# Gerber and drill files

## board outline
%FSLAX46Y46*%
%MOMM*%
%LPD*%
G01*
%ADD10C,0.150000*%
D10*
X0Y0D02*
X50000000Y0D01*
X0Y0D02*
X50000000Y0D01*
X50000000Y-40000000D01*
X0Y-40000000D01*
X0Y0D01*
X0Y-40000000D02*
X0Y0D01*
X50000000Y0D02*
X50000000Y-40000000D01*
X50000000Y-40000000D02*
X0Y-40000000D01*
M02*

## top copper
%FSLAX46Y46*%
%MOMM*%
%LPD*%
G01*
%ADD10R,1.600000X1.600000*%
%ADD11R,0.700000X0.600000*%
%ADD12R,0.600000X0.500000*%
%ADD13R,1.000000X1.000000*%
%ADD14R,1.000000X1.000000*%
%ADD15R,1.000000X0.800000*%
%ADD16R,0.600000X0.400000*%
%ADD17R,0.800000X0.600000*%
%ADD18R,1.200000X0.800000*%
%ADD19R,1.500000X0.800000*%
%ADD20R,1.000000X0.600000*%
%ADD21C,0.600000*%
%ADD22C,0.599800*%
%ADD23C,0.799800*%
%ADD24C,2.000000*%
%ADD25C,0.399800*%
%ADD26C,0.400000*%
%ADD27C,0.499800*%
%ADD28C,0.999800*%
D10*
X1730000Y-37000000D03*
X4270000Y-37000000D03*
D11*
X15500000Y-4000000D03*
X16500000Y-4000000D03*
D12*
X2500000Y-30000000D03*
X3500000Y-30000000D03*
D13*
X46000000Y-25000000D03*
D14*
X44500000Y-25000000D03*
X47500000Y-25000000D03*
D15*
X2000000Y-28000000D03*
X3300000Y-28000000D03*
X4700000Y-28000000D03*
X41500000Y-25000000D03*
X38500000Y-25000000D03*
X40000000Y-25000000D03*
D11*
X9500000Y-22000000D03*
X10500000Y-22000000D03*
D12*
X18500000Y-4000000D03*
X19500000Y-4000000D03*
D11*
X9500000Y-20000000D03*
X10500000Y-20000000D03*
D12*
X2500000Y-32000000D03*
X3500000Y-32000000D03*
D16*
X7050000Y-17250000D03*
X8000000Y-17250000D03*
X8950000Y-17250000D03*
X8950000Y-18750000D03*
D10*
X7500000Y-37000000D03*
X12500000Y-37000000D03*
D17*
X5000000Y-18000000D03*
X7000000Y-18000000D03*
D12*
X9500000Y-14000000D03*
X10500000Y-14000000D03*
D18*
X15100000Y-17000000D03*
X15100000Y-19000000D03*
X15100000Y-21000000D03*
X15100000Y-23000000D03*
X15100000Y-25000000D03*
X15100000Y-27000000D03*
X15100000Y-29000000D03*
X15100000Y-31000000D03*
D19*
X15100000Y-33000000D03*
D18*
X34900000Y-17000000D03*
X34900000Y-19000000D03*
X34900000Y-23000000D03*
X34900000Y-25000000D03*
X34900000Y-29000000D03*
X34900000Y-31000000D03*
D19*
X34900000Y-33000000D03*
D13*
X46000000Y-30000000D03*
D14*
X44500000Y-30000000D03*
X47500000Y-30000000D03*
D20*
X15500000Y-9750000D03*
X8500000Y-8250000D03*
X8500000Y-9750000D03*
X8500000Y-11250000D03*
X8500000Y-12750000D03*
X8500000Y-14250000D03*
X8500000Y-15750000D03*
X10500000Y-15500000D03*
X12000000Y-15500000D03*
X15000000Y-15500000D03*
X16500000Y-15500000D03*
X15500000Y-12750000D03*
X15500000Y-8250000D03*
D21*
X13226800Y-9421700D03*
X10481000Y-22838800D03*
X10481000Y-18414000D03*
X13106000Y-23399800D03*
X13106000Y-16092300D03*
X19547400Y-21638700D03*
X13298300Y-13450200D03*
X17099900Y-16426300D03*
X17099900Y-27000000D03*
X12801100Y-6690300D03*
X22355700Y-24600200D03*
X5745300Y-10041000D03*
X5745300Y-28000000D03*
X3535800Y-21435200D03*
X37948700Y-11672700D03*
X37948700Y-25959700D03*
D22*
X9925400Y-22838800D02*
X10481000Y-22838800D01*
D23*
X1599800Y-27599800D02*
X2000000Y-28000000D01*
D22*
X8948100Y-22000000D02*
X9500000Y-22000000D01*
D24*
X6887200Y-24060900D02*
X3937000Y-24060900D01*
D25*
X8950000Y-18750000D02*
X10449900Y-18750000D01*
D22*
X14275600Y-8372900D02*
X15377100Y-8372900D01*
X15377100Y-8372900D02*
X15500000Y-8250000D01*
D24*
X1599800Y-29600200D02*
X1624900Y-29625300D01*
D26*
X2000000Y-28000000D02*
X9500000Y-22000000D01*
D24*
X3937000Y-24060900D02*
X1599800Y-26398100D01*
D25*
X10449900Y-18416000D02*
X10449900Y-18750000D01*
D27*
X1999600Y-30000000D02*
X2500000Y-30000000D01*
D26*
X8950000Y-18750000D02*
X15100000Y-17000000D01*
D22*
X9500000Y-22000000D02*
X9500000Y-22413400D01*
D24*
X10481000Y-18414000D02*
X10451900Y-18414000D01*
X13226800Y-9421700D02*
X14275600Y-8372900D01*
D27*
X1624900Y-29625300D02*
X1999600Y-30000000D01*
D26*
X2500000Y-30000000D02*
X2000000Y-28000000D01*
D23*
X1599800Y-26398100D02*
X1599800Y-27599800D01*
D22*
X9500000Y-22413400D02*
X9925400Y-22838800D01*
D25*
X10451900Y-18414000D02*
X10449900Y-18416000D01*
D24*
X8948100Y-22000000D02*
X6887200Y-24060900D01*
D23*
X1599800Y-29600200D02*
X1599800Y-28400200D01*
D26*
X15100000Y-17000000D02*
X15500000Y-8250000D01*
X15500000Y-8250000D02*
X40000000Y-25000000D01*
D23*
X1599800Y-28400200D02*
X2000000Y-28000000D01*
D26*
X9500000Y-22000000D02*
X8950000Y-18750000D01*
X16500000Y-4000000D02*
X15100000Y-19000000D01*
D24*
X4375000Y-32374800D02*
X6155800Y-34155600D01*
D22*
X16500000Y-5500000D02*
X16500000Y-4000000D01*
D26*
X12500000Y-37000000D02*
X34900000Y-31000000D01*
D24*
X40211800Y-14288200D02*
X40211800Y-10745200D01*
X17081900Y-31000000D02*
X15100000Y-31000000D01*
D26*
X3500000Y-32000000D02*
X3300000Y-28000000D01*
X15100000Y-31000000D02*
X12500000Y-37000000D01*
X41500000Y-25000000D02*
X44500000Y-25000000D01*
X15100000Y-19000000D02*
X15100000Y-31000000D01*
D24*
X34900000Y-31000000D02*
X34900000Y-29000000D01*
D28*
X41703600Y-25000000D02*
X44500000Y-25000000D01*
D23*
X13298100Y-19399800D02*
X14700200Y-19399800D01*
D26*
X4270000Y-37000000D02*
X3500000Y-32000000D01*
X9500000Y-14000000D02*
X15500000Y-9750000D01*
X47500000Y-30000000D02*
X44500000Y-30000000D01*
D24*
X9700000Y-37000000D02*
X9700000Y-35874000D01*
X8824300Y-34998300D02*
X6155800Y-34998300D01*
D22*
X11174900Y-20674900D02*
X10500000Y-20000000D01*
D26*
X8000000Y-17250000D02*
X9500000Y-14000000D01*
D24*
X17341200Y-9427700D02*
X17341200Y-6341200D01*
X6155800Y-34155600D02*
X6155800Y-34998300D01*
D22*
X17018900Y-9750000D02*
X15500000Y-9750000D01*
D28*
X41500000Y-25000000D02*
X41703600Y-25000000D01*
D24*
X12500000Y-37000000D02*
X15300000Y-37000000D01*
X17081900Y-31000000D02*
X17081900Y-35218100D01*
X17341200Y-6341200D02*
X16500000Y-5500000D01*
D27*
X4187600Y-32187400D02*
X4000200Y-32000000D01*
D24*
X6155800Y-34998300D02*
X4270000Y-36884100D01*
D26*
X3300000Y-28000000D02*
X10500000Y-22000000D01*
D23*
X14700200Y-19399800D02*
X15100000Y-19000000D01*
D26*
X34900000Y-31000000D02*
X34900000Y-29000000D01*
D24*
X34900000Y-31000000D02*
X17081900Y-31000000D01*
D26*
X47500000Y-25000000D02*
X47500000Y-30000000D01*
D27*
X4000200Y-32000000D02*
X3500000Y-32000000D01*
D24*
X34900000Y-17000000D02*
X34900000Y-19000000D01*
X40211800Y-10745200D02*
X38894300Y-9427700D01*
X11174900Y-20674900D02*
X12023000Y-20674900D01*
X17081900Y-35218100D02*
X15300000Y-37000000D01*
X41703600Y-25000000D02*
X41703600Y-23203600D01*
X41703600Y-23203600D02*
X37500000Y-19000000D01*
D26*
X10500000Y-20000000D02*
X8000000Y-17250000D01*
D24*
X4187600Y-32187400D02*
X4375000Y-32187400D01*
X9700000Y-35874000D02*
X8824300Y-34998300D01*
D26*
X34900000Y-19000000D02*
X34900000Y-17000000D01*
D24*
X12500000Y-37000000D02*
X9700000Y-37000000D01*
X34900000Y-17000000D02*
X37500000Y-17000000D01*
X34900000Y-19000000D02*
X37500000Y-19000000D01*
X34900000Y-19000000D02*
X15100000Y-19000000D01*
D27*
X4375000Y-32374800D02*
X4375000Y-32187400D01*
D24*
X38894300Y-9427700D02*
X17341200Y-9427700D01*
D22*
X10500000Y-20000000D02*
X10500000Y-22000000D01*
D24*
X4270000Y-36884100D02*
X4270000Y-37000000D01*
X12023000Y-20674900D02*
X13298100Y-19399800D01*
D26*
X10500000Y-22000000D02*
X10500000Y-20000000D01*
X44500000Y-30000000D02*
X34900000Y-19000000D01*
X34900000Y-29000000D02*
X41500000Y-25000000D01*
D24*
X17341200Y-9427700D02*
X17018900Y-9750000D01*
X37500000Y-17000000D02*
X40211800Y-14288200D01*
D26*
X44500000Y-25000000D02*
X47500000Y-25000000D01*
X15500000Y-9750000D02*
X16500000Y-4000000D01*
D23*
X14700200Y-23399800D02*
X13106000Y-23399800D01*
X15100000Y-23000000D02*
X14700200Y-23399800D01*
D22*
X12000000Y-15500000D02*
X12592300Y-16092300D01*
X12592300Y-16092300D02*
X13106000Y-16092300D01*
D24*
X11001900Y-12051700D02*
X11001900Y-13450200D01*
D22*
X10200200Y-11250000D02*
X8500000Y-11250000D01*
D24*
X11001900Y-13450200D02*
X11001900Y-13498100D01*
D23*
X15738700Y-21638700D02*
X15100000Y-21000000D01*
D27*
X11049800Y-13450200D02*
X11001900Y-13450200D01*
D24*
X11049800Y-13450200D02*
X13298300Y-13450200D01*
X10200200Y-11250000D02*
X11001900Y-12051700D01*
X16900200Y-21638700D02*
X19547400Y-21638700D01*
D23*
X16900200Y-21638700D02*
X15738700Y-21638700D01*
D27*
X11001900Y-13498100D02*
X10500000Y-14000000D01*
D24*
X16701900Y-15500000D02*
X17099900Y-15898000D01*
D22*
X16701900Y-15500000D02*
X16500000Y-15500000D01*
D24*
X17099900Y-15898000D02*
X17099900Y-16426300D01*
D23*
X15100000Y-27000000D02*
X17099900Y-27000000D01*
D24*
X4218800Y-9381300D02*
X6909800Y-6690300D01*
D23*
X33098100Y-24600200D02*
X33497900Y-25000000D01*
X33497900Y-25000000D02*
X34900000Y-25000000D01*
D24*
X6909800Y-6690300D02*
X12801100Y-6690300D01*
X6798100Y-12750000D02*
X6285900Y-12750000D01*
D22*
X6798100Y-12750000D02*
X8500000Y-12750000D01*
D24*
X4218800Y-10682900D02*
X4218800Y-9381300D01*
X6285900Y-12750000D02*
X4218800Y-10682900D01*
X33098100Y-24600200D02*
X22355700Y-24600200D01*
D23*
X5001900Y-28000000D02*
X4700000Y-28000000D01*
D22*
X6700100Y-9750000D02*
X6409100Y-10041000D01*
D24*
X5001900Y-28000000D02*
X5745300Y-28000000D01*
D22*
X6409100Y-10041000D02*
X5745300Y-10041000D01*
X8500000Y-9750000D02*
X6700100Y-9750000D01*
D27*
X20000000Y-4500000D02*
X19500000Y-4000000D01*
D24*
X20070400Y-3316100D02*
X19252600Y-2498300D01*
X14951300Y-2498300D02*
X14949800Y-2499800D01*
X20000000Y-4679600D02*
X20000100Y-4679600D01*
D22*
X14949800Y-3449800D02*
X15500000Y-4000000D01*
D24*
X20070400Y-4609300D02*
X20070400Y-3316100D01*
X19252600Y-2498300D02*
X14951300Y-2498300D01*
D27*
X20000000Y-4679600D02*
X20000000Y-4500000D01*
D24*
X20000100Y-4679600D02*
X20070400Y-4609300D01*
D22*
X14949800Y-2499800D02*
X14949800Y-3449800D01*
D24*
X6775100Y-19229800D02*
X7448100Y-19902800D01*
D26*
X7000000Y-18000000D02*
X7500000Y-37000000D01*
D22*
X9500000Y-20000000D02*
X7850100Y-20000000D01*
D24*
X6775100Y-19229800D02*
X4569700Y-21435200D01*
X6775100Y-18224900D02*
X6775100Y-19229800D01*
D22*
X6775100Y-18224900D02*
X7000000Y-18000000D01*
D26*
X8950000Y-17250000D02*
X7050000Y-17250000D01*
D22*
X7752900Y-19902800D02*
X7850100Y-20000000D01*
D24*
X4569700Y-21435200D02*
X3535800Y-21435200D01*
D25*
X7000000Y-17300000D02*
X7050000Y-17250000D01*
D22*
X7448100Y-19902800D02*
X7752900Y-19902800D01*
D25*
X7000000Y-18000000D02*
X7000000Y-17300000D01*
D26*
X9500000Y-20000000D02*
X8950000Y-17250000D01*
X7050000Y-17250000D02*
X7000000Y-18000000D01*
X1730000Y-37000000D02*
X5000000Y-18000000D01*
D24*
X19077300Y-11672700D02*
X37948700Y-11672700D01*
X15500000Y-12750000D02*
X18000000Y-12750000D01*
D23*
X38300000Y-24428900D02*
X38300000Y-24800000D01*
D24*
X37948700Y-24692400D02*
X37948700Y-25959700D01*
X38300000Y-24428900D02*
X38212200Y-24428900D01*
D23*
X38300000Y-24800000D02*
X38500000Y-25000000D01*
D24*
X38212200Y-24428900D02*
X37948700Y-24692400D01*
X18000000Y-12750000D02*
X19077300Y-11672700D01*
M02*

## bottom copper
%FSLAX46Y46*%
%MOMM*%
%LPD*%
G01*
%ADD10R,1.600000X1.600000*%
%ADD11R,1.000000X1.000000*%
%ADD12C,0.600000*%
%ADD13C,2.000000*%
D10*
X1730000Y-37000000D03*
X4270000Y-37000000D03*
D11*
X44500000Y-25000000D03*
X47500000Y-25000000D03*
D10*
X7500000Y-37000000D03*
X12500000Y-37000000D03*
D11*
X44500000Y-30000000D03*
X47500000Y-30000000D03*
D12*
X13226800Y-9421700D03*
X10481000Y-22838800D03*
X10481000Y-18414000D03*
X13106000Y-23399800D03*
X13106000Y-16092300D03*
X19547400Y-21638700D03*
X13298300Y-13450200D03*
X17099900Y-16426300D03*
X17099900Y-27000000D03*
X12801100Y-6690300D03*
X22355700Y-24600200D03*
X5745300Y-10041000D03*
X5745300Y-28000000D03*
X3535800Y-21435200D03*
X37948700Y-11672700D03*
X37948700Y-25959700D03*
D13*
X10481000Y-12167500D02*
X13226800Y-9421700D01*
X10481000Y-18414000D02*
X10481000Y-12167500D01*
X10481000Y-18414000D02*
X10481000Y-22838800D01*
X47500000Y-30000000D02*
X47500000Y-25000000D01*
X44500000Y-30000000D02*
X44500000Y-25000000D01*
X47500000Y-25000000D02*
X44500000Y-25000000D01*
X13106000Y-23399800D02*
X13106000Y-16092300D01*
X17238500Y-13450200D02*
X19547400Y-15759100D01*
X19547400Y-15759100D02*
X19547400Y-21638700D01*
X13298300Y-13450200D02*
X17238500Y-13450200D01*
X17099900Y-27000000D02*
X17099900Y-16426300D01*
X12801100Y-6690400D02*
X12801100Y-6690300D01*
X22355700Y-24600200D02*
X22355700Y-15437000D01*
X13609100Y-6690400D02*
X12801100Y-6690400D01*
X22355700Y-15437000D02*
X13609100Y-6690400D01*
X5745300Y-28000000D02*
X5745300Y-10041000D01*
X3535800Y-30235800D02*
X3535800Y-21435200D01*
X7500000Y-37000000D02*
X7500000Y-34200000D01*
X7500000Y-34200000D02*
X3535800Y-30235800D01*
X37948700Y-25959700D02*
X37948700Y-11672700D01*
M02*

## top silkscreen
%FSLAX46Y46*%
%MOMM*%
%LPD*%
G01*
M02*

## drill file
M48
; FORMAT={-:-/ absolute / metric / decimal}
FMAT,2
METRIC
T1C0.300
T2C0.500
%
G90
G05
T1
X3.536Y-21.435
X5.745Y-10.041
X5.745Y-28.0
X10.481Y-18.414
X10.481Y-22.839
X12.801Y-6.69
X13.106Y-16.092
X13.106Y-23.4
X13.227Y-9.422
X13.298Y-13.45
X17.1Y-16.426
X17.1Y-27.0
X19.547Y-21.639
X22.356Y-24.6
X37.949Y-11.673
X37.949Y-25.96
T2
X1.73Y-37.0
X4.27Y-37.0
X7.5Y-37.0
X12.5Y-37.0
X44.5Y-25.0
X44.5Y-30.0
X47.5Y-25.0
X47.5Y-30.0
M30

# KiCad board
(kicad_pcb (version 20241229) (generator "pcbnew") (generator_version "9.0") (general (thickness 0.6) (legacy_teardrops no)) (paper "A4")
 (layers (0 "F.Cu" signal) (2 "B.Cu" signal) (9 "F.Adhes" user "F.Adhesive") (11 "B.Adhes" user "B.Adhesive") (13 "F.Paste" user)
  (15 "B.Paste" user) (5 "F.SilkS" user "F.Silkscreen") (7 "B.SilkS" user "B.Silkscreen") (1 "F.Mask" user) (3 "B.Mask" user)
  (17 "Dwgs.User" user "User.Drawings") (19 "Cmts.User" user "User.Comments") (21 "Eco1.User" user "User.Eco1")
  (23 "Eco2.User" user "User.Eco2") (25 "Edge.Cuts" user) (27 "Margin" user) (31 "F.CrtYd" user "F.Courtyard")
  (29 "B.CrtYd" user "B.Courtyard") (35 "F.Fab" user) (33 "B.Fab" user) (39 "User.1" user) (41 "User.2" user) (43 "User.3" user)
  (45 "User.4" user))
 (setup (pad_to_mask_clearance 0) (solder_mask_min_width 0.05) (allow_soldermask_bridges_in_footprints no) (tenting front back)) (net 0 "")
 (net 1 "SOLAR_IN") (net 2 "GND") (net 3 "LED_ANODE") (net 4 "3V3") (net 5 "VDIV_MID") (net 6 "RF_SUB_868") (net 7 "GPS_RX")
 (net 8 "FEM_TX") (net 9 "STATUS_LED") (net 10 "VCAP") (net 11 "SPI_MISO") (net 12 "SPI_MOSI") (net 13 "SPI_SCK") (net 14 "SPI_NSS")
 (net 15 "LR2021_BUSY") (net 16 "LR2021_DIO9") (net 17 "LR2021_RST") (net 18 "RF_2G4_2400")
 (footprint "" (layer "F.Cu") (at 3 37)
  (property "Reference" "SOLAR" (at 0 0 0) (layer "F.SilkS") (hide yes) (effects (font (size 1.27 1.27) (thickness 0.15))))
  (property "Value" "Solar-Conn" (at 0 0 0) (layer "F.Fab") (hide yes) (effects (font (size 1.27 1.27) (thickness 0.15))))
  (pad "1" thru_hole rect (at -1.27 0) (size 1.6 1.6) (drill 0.5) (layers "*.Cu" "*.Mask") (remove_unused_layers no) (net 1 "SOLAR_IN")
   (thermal_bridge_angle 45))
  (pad "2" thru_hole rect (at 1.27 0) (size 1.6 1.6) (drill 0.5) (layers "*.Cu" "*.Mask") (remove_unused_layers no) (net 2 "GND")
   (thermal_bridge_angle 45)))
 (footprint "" (layer "F.Cu") (at 16 4)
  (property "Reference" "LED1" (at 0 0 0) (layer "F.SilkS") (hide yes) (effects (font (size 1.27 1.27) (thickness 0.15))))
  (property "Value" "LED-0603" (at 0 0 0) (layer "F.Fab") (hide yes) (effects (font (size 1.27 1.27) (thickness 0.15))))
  (pad "A" smd rect (at -0.5 0) (size 0.7 0.6) (layers "F.Cu" "F.Mask") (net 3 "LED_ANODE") (thermal_bridge_angle 45))
  (pad "K" smd rect (at 0.5 0) (size 0.7 0.6) (layers "F.Cu" "F.Mask") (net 2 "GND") (thermal_bridge_angle 45)))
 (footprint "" (layer "F.Cu") (at 3 30)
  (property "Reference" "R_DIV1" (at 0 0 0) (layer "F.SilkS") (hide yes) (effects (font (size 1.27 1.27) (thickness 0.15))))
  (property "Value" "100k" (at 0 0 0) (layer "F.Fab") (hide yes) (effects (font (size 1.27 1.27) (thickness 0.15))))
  (pad "1" smd rect (at -0.5 0) (size 0.6 0.5) (layers "F.Cu" "F.Mask") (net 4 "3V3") (thermal_bridge_angle 45))
  (pad "2" smd rect (at 0.5 0) (size 0.6 0.5) (layers "F.Cu" "F.Mask") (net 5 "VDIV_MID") (thermal_bridge_angle 45)))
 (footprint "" (layer "F.Cu") (at 46 25)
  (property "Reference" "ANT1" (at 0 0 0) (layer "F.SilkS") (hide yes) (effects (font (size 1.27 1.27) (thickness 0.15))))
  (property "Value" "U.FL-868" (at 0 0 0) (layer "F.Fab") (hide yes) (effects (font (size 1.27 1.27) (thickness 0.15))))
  (pad "1" smd rect (at 0 0) (size 1 1) (layers "F.Cu" "F.Mask") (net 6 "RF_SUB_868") (thermal_bridge_angle 45))
  (pad "2" thru_hole rect (at -1.5 0) (size 1 1) (drill 0.5) (layers "*.Cu" "*.Mask") (remove_unused_layers no) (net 2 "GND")
   (thermal_bridge_angle 45))
  (pad "3" thru_hole rect (at 1.5 0) (size 1 1) (drill 0.5) (layers "*.Cu" "*.Mask") (remove_unused_layers no) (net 2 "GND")
   (thermal_bridge_angle 45)))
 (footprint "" (layer "F.Cu") (at 4 28)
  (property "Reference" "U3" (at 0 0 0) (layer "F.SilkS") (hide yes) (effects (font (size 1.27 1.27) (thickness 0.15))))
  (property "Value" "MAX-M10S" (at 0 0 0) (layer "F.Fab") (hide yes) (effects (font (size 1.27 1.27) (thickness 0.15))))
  (pad "1" smd rect (at -2 0) (size 1 0.8) (layers "F.Cu" "F.Mask") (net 4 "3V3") (thermal_bridge_angle 45))
  (pad "2" smd rect (at -0.7 0) (size 1 0.8) (layers "F.Cu" "F.Mask") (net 2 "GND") (thermal_bridge_angle 45))
  (pad "3" smd rect (at 0.7 0) (size 1 0.8) (layers "F.Cu" "F.Mask") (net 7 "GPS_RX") (thermal_bridge_angle 45)))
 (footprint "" (layer "F.Cu") (at 40 25)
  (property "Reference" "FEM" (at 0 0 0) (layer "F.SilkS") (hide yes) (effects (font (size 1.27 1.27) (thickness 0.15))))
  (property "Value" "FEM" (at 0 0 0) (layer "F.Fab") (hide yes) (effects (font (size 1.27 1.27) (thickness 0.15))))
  (pad "GND" smd rect (at 1.5 0) (size 1 0.8) (layers "F.Cu" "F.Mask") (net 2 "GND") (thermal_bridge_angle 45))
  (pad "TX" smd rect (at -1.5 0) (size 1 0.8) (layers "F.Cu" "F.Mask") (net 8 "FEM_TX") (thermal_bridge_angle 45))
  (pad "VCC" smd rect (at 0 0) (size 1 0.8) (layers "F.Cu" "F.Mask") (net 4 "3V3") (thermal_bridge_angle 45)))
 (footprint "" (layer "F.Cu") (at 10 22)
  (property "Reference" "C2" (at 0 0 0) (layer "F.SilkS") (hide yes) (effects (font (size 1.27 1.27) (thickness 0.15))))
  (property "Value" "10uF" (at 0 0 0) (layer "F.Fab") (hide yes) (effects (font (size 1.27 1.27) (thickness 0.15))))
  (pad "1" smd rect (at -0.5 0) (size 0.7 0.6) (layers "F.Cu" "F.Mask") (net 4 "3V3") (thermal_bridge_angle 45))
  (pad "2" smd rect (at 0.5 0) (size 0.7 0.6) (layers "F.Cu" "F.Mask") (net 2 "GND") (thermal_bridge_angle 45)))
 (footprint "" (layer "F.Cu") (at 19 4)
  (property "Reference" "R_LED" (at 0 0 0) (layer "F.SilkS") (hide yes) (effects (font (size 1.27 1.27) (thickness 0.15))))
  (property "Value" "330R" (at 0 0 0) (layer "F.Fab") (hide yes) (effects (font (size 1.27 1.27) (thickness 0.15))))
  (pad "1" smd rect (at -0.5 0) (size 0.6 0.5) (layers "F.Cu" "F.Mask") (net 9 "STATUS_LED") (thermal_bridge_angle 45))
  (pad "2" smd rect (at 0.5 0) (size 0.6 0.5) (layers "F.Cu" "F.Mask") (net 3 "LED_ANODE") (thermal_bridge_angle 45)))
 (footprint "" (layer "F.Cu") (at 10 20)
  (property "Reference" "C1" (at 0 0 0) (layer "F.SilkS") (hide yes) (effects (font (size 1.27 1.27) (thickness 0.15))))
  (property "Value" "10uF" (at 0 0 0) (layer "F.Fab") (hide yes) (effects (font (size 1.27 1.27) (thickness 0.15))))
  (pad "1" smd rect (at -0.5 0) (size 0.7 0.6) (layers "F.Cu" "F.Mask") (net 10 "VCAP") (thermal_bridge_angle 45))
  (pad "2" smd rect (at 0.5 0) (size 0.7 0.6) (layers "F.Cu" "F.Mask") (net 2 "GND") (thermal_bridge_angle 45)))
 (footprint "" (layer "F.Cu") (at 3 32)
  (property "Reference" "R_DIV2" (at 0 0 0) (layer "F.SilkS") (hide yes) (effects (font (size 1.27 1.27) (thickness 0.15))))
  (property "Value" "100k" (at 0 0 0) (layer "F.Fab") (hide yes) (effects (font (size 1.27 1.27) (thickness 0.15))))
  (pad "1" smd rect (at -0.5 0) (size 0.6 0.5) (layers "F.Cu" "F.Mask") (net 5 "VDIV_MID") (thermal_bridge_angle 45))
  (pad "2" smd rect (at 0.5 0) (size 0.6 0.5) (layers "F.Cu" "F.Mask") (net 2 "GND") (thermal_bridge_angle 45)))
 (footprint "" (layer "F.Cu") (at 8 18)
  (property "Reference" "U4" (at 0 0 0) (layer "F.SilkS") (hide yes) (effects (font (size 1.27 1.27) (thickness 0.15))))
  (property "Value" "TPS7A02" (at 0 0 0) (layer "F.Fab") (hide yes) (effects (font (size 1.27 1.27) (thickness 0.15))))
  (pad "1" smd rect (at -0.95 -0.75) (size 0.6 0.4) (layers "F.Cu" "F.Mask") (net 10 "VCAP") (thermal_bridge_angle 45))
  (pad "2" smd rect (at 0 -0.75) (size 0.6 0.4) (layers "F.Cu" "F.Mask") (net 2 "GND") (thermal_bridge_angle 45))
  (pad "3" smd rect (at 0.95 -0.75) (size 0.6 0.4) (layers "F.Cu" "F.Mask") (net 10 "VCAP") (thermal_bridge_angle 45))
  (pad "4" smd rect (at 0.95 0.75) (size 0.6 0.4) (layers "F.Cu" "F.Mask") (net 4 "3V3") (thermal_bridge_angle 45)))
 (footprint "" (layer "F.Cu") (at 10 37)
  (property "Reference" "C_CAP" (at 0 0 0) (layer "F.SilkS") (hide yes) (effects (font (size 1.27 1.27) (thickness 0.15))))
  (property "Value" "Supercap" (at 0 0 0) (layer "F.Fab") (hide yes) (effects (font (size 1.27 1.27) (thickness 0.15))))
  (pad "1" thru_hole rect (at -2.5 0) (size 1.6 1.6) (drill 0.5) (layers "*.Cu" "*.Mask") (remove_unused_layers no) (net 10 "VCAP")
   (thermal_bridge_angle 45))
  (pad "2" thru_hole rect (at 2.5 0) (size 1.6 1.6) (drill 0.5) (layers "*.Cu" "*.Mask") (remove_unused_layers no) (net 2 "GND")
   (thermal_bridge_angle 45)))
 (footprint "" (layer "F.Cu") (at 6 18)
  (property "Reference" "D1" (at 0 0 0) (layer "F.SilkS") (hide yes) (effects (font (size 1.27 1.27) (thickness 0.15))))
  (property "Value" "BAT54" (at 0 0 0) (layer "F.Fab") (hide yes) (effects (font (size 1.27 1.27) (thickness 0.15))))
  (pad "A" smd rect (at -1 0) (size 0.8 0.6) (layers "F.Cu" "F.Mask") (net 1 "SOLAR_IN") (thermal_bridge_angle 45))
  (pad "K" smd rect (at 1 0) (size 0.8 0.6) (layers "F.Cu" "F.Mask") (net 10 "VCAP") (thermal_bridge_angle 45)))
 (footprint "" (layer "F.Cu") (at 10 14)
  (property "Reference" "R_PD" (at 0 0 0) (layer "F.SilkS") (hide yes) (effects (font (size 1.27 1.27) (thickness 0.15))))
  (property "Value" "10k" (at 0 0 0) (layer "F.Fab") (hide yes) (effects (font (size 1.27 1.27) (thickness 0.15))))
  (pad "1" smd rect (at -0.5 0) (size 0.6 0.5) (layers "F.Cu" "F.Mask") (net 2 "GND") (thermal_bridge_angle 45))
  (pad "2" smd rect (at 0.5 0) (size 0.6 0.5) (layers "F.Cu" "F.Mask") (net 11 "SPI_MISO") (thermal_bridge_angle 45)))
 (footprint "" (layer "F.Cu") (at 25 25)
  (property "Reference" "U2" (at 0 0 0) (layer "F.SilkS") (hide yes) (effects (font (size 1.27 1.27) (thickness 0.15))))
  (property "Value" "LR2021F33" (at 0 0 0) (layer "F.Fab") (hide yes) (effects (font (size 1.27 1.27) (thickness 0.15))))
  (pad "1" smd rect (at -9.9 -8) (size 1.2 0.8) (layers "F.Cu" "F.Mask") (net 4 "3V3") (thermal_bridge_angle 45))
  (pad "2" smd rect (at -9.9 -6) (size 1.2 0.8) (layers "F.Cu" "F.Mask") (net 2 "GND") (thermal_bridge_angle 45))
  (pad "3" smd rect (at -9.9 -4) (size 1.2 0.8) (layers "F.Cu" "F.Mask") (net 11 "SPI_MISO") (thermal_bridge_angle 45))
  (pad "4" smd rect (at -9.9 -2) (size 1.2 0.8) (layers "F.Cu" "F.Mask") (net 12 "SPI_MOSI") (thermal_bridge_angle 45))
  (pad "5" smd rect (at -9.9 0) (size 1.2 0.8) (layers "F.Cu" "F.Mask") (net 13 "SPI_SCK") (thermal_bridge_angle 45))
  (pad "6" smd rect (at -9.9 2) (size 1.2 0.8) (layers "F.Cu" "F.Mask") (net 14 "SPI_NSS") (thermal_bridge_angle 45))
  (pad "7" smd rect (at -9.9 4) (size 1.2 0.8) (layers "F.Cu" "F.Mask") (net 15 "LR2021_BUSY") (thermal_bridge_angle 45))
  (pad "8" smd rect (at -9.9 6) (size 1.2 0.8) (layers "F.Cu" "F.Mask") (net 2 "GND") (thermal_bridge_angle 45))
  (pad "9" smd rect (at -9.9 8) (size 1.5 0.8) (layers "F.Cu" "F.Mask") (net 6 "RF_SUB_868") (thermal_bridge_angle 45))
  (pad "10" smd rect (at 9.9 -8) (size 1.2 0.8) (layers "F.Cu" "F.Mask") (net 2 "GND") (thermal_bridge_angle 45))
  (pad "11" smd rect (at 9.9 -6) (size 1.2 0.8) (layers "F.Cu" "F.Mask") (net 2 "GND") (thermal_bridge_angle 45))
  (pad "13" smd rect (at 9.9 -2) (size 1.2 0.8) (layers "F.Cu" "F.Mask") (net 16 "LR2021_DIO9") (thermal_bridge_angle 45))
  (pad "14" smd rect (at 9.9 0) (size 1.2 0.8) (layers "F.Cu" "F.Mask") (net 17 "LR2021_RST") (thermal_bridge_angle 45))
  (pad "16" smd rect (at 9.9 4) (size 1.2 0.8) (layers "F.Cu" "F.Mask") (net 2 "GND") (thermal_bridge_angle 45))
  (pad "17" smd rect (at 9.9 6) (size 1.2 0.8) (layers "F.Cu" "F.Mask") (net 2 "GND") (thermal_bridge_angle 45))
  (pad "18" smd rect (at 9.9 8) (size 1.5 0.8) (layers "F.Cu" "F.Mask") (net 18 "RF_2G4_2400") (thermal_bridge_angle 45)))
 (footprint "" (layer "F.Cu") (at 46 30)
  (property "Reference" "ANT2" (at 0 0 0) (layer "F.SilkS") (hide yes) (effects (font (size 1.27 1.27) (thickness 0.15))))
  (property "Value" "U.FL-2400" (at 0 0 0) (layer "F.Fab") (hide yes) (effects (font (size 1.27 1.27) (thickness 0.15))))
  (pad "1" smd rect (at 0 0) (size 1 1) (layers "F.Cu" "F.Mask") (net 18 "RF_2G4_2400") (thermal_bridge_angle 45))
  (pad "2" thru_hole rect (at -1.5 0) (size 1 1) (drill 0.5) (layers "*.Cu" "*.Mask") (remove_unused_layers no) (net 2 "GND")
   (thermal_bridge_angle 45))
  (pad "3" thru_hole rect (at 1.5 0) (size 1 1) (drill 0.5) (layers "*.Cu" "*.Mask") (remove_unused_layers no) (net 2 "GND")
   (thermal_bridge_angle 45)))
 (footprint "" (layer "F.Cu") (at 12 12)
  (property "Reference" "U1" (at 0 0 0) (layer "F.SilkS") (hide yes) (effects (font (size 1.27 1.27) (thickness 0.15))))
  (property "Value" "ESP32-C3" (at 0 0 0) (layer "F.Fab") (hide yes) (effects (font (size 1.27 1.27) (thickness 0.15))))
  (pad "GND" smd rect (at 3.5 -2.25) (size 1 0.6) (layers "F.Cu" "F.Mask") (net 2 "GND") (thermal_bridge_angle 45))
  (pad "GPIO0" smd rect (at -3.5 -3.75) (size 1 0.6) (layers "F.Cu" "F.Mask") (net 5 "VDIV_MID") (thermal_bridge_angle 45))
  (pad "GPIO1" smd rect (at -3.5 -2.25) (size 1 0.6) (layers "F.Cu" "F.Mask") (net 7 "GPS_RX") (thermal_bridge_angle 45))
  (pad "GPIO2" smd rect (at -3.5 -0.75) (size 1 0.6) (layers "F.Cu" "F.Mask") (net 11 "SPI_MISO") (thermal_bridge_angle 45))
  (pad "GPIO3" smd rect (at -3.5 0.75) (size 1 0.6) (layers "F.Cu" "F.Mask") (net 17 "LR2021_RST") (thermal_bridge_angle 45))
  (pad "GPIO4" smd rect (at -3.5 2.25) (size 1 0.6) (layers "F.Cu" "F.Mask") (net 15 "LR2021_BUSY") (thermal_bridge_angle 45))
  (pad "GPIO5" smd rect (at -3.5 3.75) (size 1 0.6) (layers "F.Cu" "F.Mask") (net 16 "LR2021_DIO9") (thermal_bridge_angle 45))
  (pad "GPIO6" smd rect (at -1.5 3.5) (size 1 0.6) (layers "F.Cu" "F.Mask") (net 13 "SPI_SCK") (thermal_bridge_angle 45))
  (pad "GPIO7" smd rect (at 0 3.5) (size 1 0.6) (layers "F.Cu" "F.Mask") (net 12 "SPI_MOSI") (thermal_bridge_angle 45))
  (pad "GPIO9" smd rect (at 3 3.5) (size 1 0.6) (layers "F.Cu" "F.Mask") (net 9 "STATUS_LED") (thermal_bridge_angle 45))
  (pad "GPIO10" smd rect (at 4.5 3.5) (size 1 0.6) (layers "F.Cu" "F.Mask") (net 14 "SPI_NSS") (thermal_bridge_angle 45))
  (pad "GPIO19" smd rect (at 3.5 0.75) (size 1 0.6) (layers "F.Cu" "F.Mask") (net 8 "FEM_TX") (thermal_bridge_angle 45))
  (pad "VCC" smd rect (at 3.5 -3.75) (size 1 0.6) (layers "F.Cu" "F.Mask") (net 4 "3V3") (thermal_bridge_angle 45)))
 (gr_line (start 0 0) (end 50 0) (stroke (width 0.15) (type default)) (layer "Edge.Cuts"))
 (gr_rect (start 0 0) (end 50 40) (stroke (width 0.15) (type default)) (fill no) (layer "Edge.Cuts"))
 (gr_line (start 0 40) (end 0 0) (stroke (width 0.15) (type default)) (layer "Edge.Cuts"))
 (gr_line (start 50 0) (end 50 40) (stroke (width 0.15) (type default)) (layer "Edge.Cuts"))
 (gr_line (start 50 40) (end 0 40) (stroke (width 0.15) (type default)) (layer "Edge.Cuts"))
 (segment (start 9.9254 22.8388) (end 10.481 22.8388) (width 0.5998) (layer "F.Cu") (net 4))
 (segment (start 1.5998 27.5998) (end 2 28) (width 0.7998) (layer "F.Cu") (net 4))
 (segment (start 8.9481 22) (end 9.5 22) (width 0.5998) (layer "F.Cu") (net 4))
 (segment (start 6.8872 24.0609) (end 3.937 24.0609) (width 2) (layer "F.Cu") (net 4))
 (segment (start 8.95 18.75) (end 10.4499 18.75) (width 0.3998) (layer "F.Cu") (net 4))
 (segment (start 14.2756 8.3729) (end 15.3771 8.3729) (width 0.5998) (layer "F.Cu") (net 4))
 (segment (start 15.3771 8.3729) (end 15.5 8.25) (width 0.5998) (layer "F.Cu") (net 4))
 (segment (start 1.5998 29.6002) (end 1.6249 29.6253) (width 2) (layer "F.Cu") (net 4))
 (segment (start 2 28) (end 9.5 22) (width 0.4) (layer "F.Cu") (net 4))
 (segment (start 3.937 24.0609) (end 1.5998 26.3981) (width 2) (layer "F.Cu") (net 4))
 (segment (start 10.4499 18.416) (end 10.4499 18.75) (width 0.3998) (layer "F.Cu") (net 4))
 (segment (start 1.9996 30) (end 2.5 30) (width 0.4998) (layer "F.Cu") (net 4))
 (segment (start 8.95 18.75) (end 15.1 17) (width 0.4) (layer "F.Cu") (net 4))
 (segment (start 9.5 22) (end 9.5 22.4134) (width 0.5998) (layer "F.Cu") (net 4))
 (segment (start 10.481 18.414) (end 10.4519 18.414) (width 2) (layer "F.Cu") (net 4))
 (segment (start 13.2268 9.4217) (end 14.2756 8.3729) (width 2) (layer "F.Cu") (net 4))
 (segment (start 1.6249 29.6253) (end 1.9996 30) (width 0.4998) (layer "F.Cu") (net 4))
 (segment (start 2.5 30) (end 2 28) (width 0.4) (layer "F.Cu") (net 4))
 (segment (start 1.5998 26.3981) (end 1.5998 27.5998) (width 0.7998) (layer "F.Cu") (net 4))
 (segment (start 9.5 22.4134) (end 9.9254 22.8388) (width 0.5998) (layer "F.Cu") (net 4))
 (segment (start 10.4519 18.414) (end 10.4499 18.416) (width 0.3998) (layer "F.Cu") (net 4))
 (segment (start 8.9481 22) (end 6.8872 24.0609) (width 2) (layer "F.Cu") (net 4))
 (segment (start 1.5998 29.6002) (end 1.5998 28.4002) (width 0.7998) (layer "F.Cu") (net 4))
 (segment (start 15.1 17) (end 15.5 8.25) (width 0.4) (layer "F.Cu") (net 4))
 (segment (start 15.5 8.25) (end 40 25) (width 0.4) (layer "F.Cu") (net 4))
 (segment (start 1.5998 28.4002) (end 2 28) (width 0.7998) (layer "F.Cu") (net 4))
 (segment (start 9.5 22) (end 8.95 18.75) (width 0.4) (layer "F.Cu") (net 4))
 (via (at 13.2268 9.4217) (size 0.6) (drill 0.3) (layers "F.Cu" "B.Cu") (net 4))
 (via (at 10.481 22.8388) (size 0.6) (drill 0.3) (layers "F.Cu" "B.Cu") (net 4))
 (via (at 10.481 18.414) (size 0.6) (drill 0.3) (layers "F.Cu" "B.Cu") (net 4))
 (segment (start 10.481 12.1675) (end 13.2268 9.4217) (width 2) (layer "B.Cu") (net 4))
 (segment (start 10.481 18.414) (end 10.481 12.1675) (width 2) (layer "B.Cu") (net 4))
 (segment (start 10.481 18.414) (end 10.481 22.8388) (width 2) (layer "B.Cu") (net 4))
 (segment (start 16.5 4) (end 15.1 19) (width 0.4) (layer "F.Cu") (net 2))
 (segment (start 4.375 32.3748) (end 6.1558 34.1556) (width 2) (layer "F.Cu") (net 2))
 (segment (start 16.5 5.5) (end 16.5 4) (width 0.5998) (layer "F.Cu") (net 2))
 (segment (start 12.5 37) (end 34.9 31) (width 0.4) (layer "F.Cu") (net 2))
 (segment (start 40.2118 14.2882) (end 40.2118 10.7452) (width 2) (layer "F.Cu") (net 2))
 (segment (start 17.0819 31) (end 15.1 31) (width 2) (layer "F.Cu") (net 2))
 (segment (start 3.5 32) (end 3.3 28) (width 0.4) (layer "F.Cu") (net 2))
 (segment (start 15.1 31) (end 12.5 37) (width 0.4) (layer "F.Cu") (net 2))
 (segment (start 41.5 25) (end 44.5 25) (width 0.4) (layer "F.Cu") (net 2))
 (segment (start 15.1 19) (end 15.1 31) (width 0.4) (layer "F.Cu") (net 2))
 (segment (start 34.9 31) (end 34.9 29) (width 2) (layer "F.Cu") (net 2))
 (segment (start 41.7036 25) (end 44.5 25) (width 0.9998) (layer "F.Cu") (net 2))
 (segment (start 13.2981 19.3998) (end 14.7002 19.3998) (width 0.7998) (layer "F.Cu") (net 2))
 (segment (start 4.27 37) (end 3.5 32) (width 0.4) (layer "F.Cu") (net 2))
 (segment (start 9.5 14) (end 15.5 9.75) (width 0.4) (layer "F.Cu") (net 2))
 (segment (start 47.5 30) (end 44.5 30) (width 0.4) (layer "F.Cu") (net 2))
 (segment (start 9.7 37) (end 9.7 35.874) (width 2) (layer "F.Cu") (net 2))
 (segment (start 8.8243 34.9983) (end 6.1558 34.9983) (width 2) (layer "F.Cu") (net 2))
 (segment (start 11.1749 20.6749) (end 10.5 20) (width 0.5998) (layer "F.Cu") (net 2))
 (segment (start 8 17.25) (end 9.5 14) (width 0.4) (layer "F.Cu") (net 2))
 (segment (start 17.3412 9.4277) (end 17.3412 6.3412) (width 2) (layer "F.Cu") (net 2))
 (segment (start 6.1558 34.1556) (end 6.1558 34.9983) (width 2) (layer "F.Cu") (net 2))
 (segment (start 17.0189 9.75) (end 15.5 9.75) (width 0.5998) (layer "F.Cu") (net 2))
 (segment (start 41.5 25) (end 41.7036 25) (width 0.9998) (layer "F.Cu") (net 2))
 (segment (start 12.5 37) (end 15.3 37) (width 2) (layer "F.Cu") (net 2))
 (segment (start 17.0819 31) (end 17.0819 35.2181) (width 2) (layer "F.Cu") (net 2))
 (segment (start 17.3412 6.3412) (end 16.5 5.5) (width 2) (layer "F.Cu") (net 2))
 (segment (start 4.1876 32.1874) (end 4.0002 32) (width 0.4998) (layer "F.Cu") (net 2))
 (segment (start 6.1558 34.9983) (end 4.27 36.8841) (width 2) (layer "F.Cu") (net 2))
 (segment (start 3.3 28) (end 10.5 22) (width 0.4) (layer "F.Cu") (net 2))
 (segment (start 14.7002 19.3998) (end 15.1 19) (width 0.7998) (layer "F.Cu") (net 2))
 (segment (start 34.9 31) (end 34.9 29) (width 0.4) (layer "F.Cu") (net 2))
 (segment (start 34.9 31) (end 17.0819 31) (width 2) (layer "F.Cu") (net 2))
 (segment (start 47.5 25) (end 47.5 30) (width 0.4) (layer "F.Cu") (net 2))
 (segment (start 4.0002 32) (end 3.5 32) (width 0.4998) (layer "F.Cu") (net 2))
 (segment (start 34.9 17) (end 34.9 19) (width 2) (layer "F.Cu") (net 2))
 (segment (start 40.2118 10.7452) (end 38.8943 9.4277) (width 2) (layer "F.Cu") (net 2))
 (segment (start 11.1749 20.6749) (end 12.023 20.6749) (width 2) (layer "F.Cu") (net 2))
 (segment (start 17.0819 35.2181) (end 15.3 37) (width 2) (layer "F.Cu") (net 2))
 (segment (start 41.7036 25) (end 41.7036 23.2036) (width 2) (layer "F.Cu") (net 2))
 (segment (start 41.7036 23.2036) (end 37.5 19) (width 2) (layer "F.Cu") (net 2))
 (segment (start 10.5 20) (end 8 17.25) (width 0.4) (layer "F.Cu") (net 2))
 (segment (start 4.1876 32.1874) (end 4.375 32.1874) (width 2) (layer "F.Cu") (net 2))
 (segment (start 9.7 35.874) (end 8.8243 34.9983) (width 2) (layer "F.Cu") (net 2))
 (segment (start 34.9 19) (end 34.9 17) (width 0.4) (layer "F.Cu") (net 2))
 (segment (start 12.5 37) (end 9.7 37) (width 2) (layer "F.Cu") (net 2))
 (segment (start 34.9 17) (end 37.5 17) (width 2) (layer "F.Cu") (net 2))
 (segment (start 34.9 19) (end 37.5 19) (width 2) (layer "F.Cu") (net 2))
 (segment (start 34.9 19) (end 15.1 19) (width 2) (layer "F.Cu") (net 2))
 (segment (start 4.375 32.3748) (end 4.375 32.1874) (width 0.4998) (layer "F.Cu") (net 2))
 (segment (start 38.8943 9.4277) (end 17.3412 9.4277) (width 2) (layer "F.Cu") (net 2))
 (segment (start 10.5 20) (end 10.5 22) (width 0.5998) (layer "F.Cu") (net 2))
 (segment (start 4.27 36.8841) (end 4.27 37) (width 2) (layer "F.Cu") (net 2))
 (segment (start 12.023 20.6749) (end 13.2981 19.3998) (width 2) (layer "F.Cu") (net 2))
 (segment (start 10.5 22) (end 10.5 20) (width 0.4) (layer "F.Cu") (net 2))
 (segment (start 44.5 30) (end 34.9 19) (width 0.4) (layer "F.Cu") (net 2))
 (segment (start 34.9 29) (end 41.5 25) (width 0.4) (layer "F.Cu") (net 2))
 (segment (start 17.3412 9.4277) (end 17.0189 9.75) (width 2) (layer "F.Cu") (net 2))
 (segment (start 37.5 17) (end 40.2118 14.2882) (width 2) (layer "F.Cu") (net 2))
 (segment (start 44.5 25) (end 47.5 25) (width 0.4) (layer "F.Cu") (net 2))
 (segment (start 15.5 9.75) (end 16.5 4) (width 0.4) (layer "F.Cu") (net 2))
 (segment (start 47.5 30) (end 47.5 25) (width 2) (layer "B.Cu") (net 2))
 (segment (start 44.5 30) (end 44.5 25) (width 2) (layer "B.Cu") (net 2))
 (segment (start 47.5 25) (end 44.5 25) (width 2) (layer "B.Cu") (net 2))
 (segment (start 14.7002 23.3998) (end 13.106 23.3998) (width 0.7998) (layer "F.Cu") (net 12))
 (segment (start 15.1 23) (end 14.7002 23.3998) (width 0.7998) (layer "F.Cu") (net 12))
 (segment (start 12 15.5) (end 12.5923 16.0923) (width 0.5998) (layer "F.Cu") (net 12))
 (segment (start 12.5923 16.0923) (end 13.106 16.0923) (width 0.5998) (layer "F.Cu") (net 12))
 (via (at 13.106 23.3998) (size 0.6) (drill 0.3) (layers "F.Cu" "B.Cu") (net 12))
 (via (at 13.106 16.0923) (size 0.6) (drill 0.3) (layers "F.Cu" "B.Cu") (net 12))
 (segment (start 13.106 23.3998) (end 13.106 16.0923) (width 2) (layer "B.Cu") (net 12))
 (segment (start 11.0019 12.0517) (end 11.0019 13.4502) (width 2) (layer "F.Cu") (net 11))
 (segment (start 10.2002 11.25) (end 8.5 11.25) (width 0.5998) (layer "F.Cu") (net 11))
 (segment (start 11.0019 13.4502) (end 11.0019 13.4981) (width 2) (layer "F.Cu") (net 11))
 (segment (start 15.7387 21.6387) (end 15.1 21) (width 0.7998) (layer "F.Cu") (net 11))
 (segment (start 11.0498 13.4502) (end 11.0019 13.4502) (width 0.4998) (layer "F.Cu") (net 11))
 (segment (start 11.0498 13.4502) (end 13.2983 13.4502) (width 2) (layer "F.Cu") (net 11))
 (segment (start 10.2002 11.25) (end 11.0019 12.0517) (width 2) (layer "F.Cu") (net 11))
 (segment (start 16.9002 21.6387) (end 19.5474 21.6387) (width 2) (layer "F.Cu") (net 11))
 (segment (start 16.9002 21.6387) (end 15.7387 21.6387) (width 0.7998) (layer "F.Cu") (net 11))
 (segment (start 11.0019 13.4981) (end 10.5 14) (width 0.4998) (layer "F.Cu") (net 11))
 (via (at 19.5474 21.6387) (size 0.6) (drill 0.3) (layers "F.Cu" "B.Cu") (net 11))
 (via (at 13.2983 13.4502) (size 0.6) (drill 0.3) (layers "F.Cu" "B.Cu") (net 11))
 (segment (start 17.2385 13.4502) (end 19.5474 15.7591) (width 2) (layer "B.Cu") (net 11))
 (segment (start 19.5474 15.7591) (end 19.5474 21.6387) (width 2) (layer "B.Cu") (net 11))
 (segment (start 13.2983 13.4502) (end 17.2385 13.4502) (width 2) (layer "B.Cu") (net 11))
 (segment (start 16.7019 15.5) (end 17.0999 15.898) (width 2) (layer "F.Cu") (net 14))
 (segment (start 16.7019 15.5) (end 16.5 15.5) (width 0.5998) (layer "F.Cu") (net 14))
 (segment (start 17.0999 15.898) (end 17.0999 16.4263) (width 2) (layer "F.Cu") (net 14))
 (segment (start 15.1 27) (end 17.0999 27) (width 0.7998) (layer "F.Cu") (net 14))
 (via (at 17.0999 16.4263) (size 0.6) (drill 0.3) (layers "F.Cu" "B.Cu") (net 14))
 (via (at 17.0999 27) (size 0.6) (drill 0.3) (layers "F.Cu" "B.Cu") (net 14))
 (segment (start 17.0999 27) (end 17.0999 16.4263) (width 2) (layer "B.Cu") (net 14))
 (segment (start 4.2188 9.3813) (end 6.9098 6.6903) (width 2) (layer "F.Cu") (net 17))
 (segment (start 33.0981 24.6002) (end 33.4979 25) (width 0.7998) (layer "F.Cu") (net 17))
 (segment (start 33.4979 25) (end 34.9 25) (width 0.7998) (layer "F.Cu") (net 17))
 (segment (start 6.9098 6.6903) (end 12.8011 6.6903) (width 2) (layer "F.Cu") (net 17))
 (segment (start 6.7981 12.75) (end 6.2859 12.75) (width 2) (layer "F.Cu") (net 17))
 (segment (start 6.7981 12.75) (end 8.5 12.75) (width 0.5998) (layer "F.Cu") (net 17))
 (segment (start 4.2188 10.6829) (end 4.2188 9.3813) (width 2) (layer "F.Cu") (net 17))
 (segment (start 6.2859 12.75) (end 4.2188 10.6829) (width 2) (layer "F.Cu") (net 17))
 (segment (start 33.0981 24.6002) (end 22.3557 24.6002) (width 2) (layer "F.Cu") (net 17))
 (via (at 12.8011 6.6903) (size 0.6) (drill 0.3) (layers "F.Cu" "B.Cu") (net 17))
 (via (at 22.3557 24.6002) (size 0.6) (drill 0.3) (layers "F.Cu" "B.Cu") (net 17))
 (segment (start 12.8011 6.6904) (end 12.8011 6.6903) (width 2) (layer "B.Cu") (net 17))
 (segment (start 22.3557 24.6002) (end 22.3557 15.437) (width 2) (layer "B.Cu") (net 17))
 (segment (start 13.6091 6.6904) (end 12.8011 6.6904) (width 2) (layer "B.Cu") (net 17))
 (segment (start 22.3557 15.437) (end 13.6091 6.6904) (width 2) (layer "B.Cu") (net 17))
 (segment (start 5.0019 28) (end 4.7 28) (width 0.7998) (layer "F.Cu") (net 7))
 (segment (start 6.7001 9.75) (end 6.4091 10.041) (width 0.5998) (layer "F.Cu") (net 7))
 (segment (start 5.0019 28) (end 5.7453 28) (width 2) (layer "F.Cu") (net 7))
 (segment (start 6.4091 10.041) (end 5.7453 10.041) (width 0.5998) (layer "F.Cu") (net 7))
 (segment (start 8.5 9.75) (end 6.7001 9.75) (width 0.5998) (layer "F.Cu") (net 7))
 (via (at 5.7453 10.041) (size 0.6) (drill 0.3) (layers "F.Cu" "B.Cu") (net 7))
 (via (at 5.7453 28) (size 0.6) (drill 0.3) (layers "F.Cu" "B.Cu") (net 7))
 (segment (start 5.7453 28) (end 5.7453 10.041) (width 2) (layer "B.Cu") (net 7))
 (segment (start 20 4.5) (end 19.5 4) (width 0.4998) (layer "F.Cu") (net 3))
 (segment (start 20.0704 3.3161) (end 19.2526 2.4983) (width 2) (layer "F.Cu") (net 3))
 (segment (start 14.9513 2.4983) (end 14.9498 2.4998) (width 2) (layer "F.Cu") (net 3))
 (segment (start 20 4.6796) (end 20.0001 4.6796) (width 2) (layer "F.Cu") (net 3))
 (segment (start 14.9498 3.4498) (end 15.5 4) (width 0.5998) (layer "F.Cu") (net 3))
 (segment (start 20.0704 4.6093) (end 20.0704 3.3161) (width 2) (layer "F.Cu") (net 3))
 (segment (start 19.2526 2.4983) (end 14.9513 2.4983) (width 2) (layer "F.Cu") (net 3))
 (segment (start 20 4.6796) (end 20 4.5) (width 0.4998) (layer "F.Cu") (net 3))
 (segment (start 20.0001 4.6796) (end 20.0704 4.6093) (width 2) (layer "F.Cu") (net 3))
 (segment (start 14.9498 2.4998) (end 14.9498 3.4498) (width 0.5998) (layer "F.Cu") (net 3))
 (segment (start 6.7751 19.2298) (end 7.4481 19.9028) (width 2) (layer "F.Cu") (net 10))
 (segment (start 7 18) (end 7.5 37) (width 0.4) (layer "F.Cu") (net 10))
 (segment (start 9.5 20) (end 7.8501 20) (width 0.5998) (layer "F.Cu") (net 10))
 (segment (start 6.7751 19.2298) (end 4.5697 21.4352) (width 2) (layer "F.Cu") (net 10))
 (segment (start 6.7751 18.2249) (end 6.7751 19.2298) (width 2) (layer "F.Cu") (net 10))
 (segment (start 6.7751 18.2249) (end 7 18) (width 0.5998) (layer "F.Cu") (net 10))
 (segment (start 8.95 17.25) (end 7.05 17.25) (width 0.4) (layer "F.Cu") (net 10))
 (segment (start 7.7529 19.9028) (end 7.8501 20) (width 0.5998) (layer "F.Cu") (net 10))
 (segment (start 4.5697 21.4352) (end 3.5358 21.4352) (width 2) (layer "F.Cu") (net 10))
 (segment (start 7 17.3) (end 7.05 17.25) (width 0.3998) (layer "F.Cu") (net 10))
 (segment (start 7.4481 19.9028) (end 7.7529 19.9028) (width 0.5998) (layer "F.Cu") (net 10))
 (segment (start 7 18) (end 7 17.3) (width 0.3998) (layer "F.Cu") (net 10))
 (segment (start 9.5 20) (end 8.95 17.25) (width 0.4) (layer "F.Cu") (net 10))
 (segment (start 7.05 17.25) (end 7 18) (width 0.4) (layer "F.Cu") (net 10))
 (via (at 3.5358 21.4352) (size 0.6) (drill 0.3) (layers "F.Cu" "B.Cu") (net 10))
 (segment (start 3.5358 30.2358) (end 3.5358 21.4352) (width 2) (layer "B.Cu") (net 10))
 (segment (start 7.5 37) (end 7.5 34.2) (width 2) (layer "B.Cu") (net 10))
 (segment (start 7.5 34.2) (end 3.5358 30.2358) (width 2) (layer "B.Cu") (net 10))
 (segment (start 1.73 37) (end 5 18) (width 0.4) (layer "F.Cu") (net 1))
 (segment (start 19.0773 11.6727) (end 37.9487 11.6727) (width 2) (layer "F.Cu") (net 8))
 (segment (start 15.5 12.75) (end 18 12.75) (width 2) (layer "F.Cu") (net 8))
 (segment (start 38.3 24.4289) (end 38.3 24.8) (width 0.7998) (layer "F.Cu") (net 8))
 (segment (start 37.9487 24.6924) (end 37.9487 25.9597) (width 2) (layer "F.Cu") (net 8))
 (segment (start 38.3 24.4289) (end 38.2122 24.4289) (width 2) (layer "F.Cu") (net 8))
 (segment (start 38.3 24.8) (end 38.5 25) (width 0.7998) (layer "F.Cu") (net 8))
 (segment (start 38.2122 24.4289) (end 37.9487 24.6924) (width 2) (layer "F.Cu") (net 8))
 (segment (start 18 12.75) (end 19.0773 11.6727) (width 2) (layer "F.Cu") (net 8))
 (via (at 37.9487 11.6727) (size 0.6) (drill 0.3) (layers "F.Cu" "B.Cu") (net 8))
 (via (at 37.9487 25.9597) (size 0.6) (drill 0.3) (layers "F.Cu" "B.Cu") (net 8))
 (segment (start 37.9487 25.9597) (end 37.9487 11.6727) (width 2) (layer "B.Cu") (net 8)))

